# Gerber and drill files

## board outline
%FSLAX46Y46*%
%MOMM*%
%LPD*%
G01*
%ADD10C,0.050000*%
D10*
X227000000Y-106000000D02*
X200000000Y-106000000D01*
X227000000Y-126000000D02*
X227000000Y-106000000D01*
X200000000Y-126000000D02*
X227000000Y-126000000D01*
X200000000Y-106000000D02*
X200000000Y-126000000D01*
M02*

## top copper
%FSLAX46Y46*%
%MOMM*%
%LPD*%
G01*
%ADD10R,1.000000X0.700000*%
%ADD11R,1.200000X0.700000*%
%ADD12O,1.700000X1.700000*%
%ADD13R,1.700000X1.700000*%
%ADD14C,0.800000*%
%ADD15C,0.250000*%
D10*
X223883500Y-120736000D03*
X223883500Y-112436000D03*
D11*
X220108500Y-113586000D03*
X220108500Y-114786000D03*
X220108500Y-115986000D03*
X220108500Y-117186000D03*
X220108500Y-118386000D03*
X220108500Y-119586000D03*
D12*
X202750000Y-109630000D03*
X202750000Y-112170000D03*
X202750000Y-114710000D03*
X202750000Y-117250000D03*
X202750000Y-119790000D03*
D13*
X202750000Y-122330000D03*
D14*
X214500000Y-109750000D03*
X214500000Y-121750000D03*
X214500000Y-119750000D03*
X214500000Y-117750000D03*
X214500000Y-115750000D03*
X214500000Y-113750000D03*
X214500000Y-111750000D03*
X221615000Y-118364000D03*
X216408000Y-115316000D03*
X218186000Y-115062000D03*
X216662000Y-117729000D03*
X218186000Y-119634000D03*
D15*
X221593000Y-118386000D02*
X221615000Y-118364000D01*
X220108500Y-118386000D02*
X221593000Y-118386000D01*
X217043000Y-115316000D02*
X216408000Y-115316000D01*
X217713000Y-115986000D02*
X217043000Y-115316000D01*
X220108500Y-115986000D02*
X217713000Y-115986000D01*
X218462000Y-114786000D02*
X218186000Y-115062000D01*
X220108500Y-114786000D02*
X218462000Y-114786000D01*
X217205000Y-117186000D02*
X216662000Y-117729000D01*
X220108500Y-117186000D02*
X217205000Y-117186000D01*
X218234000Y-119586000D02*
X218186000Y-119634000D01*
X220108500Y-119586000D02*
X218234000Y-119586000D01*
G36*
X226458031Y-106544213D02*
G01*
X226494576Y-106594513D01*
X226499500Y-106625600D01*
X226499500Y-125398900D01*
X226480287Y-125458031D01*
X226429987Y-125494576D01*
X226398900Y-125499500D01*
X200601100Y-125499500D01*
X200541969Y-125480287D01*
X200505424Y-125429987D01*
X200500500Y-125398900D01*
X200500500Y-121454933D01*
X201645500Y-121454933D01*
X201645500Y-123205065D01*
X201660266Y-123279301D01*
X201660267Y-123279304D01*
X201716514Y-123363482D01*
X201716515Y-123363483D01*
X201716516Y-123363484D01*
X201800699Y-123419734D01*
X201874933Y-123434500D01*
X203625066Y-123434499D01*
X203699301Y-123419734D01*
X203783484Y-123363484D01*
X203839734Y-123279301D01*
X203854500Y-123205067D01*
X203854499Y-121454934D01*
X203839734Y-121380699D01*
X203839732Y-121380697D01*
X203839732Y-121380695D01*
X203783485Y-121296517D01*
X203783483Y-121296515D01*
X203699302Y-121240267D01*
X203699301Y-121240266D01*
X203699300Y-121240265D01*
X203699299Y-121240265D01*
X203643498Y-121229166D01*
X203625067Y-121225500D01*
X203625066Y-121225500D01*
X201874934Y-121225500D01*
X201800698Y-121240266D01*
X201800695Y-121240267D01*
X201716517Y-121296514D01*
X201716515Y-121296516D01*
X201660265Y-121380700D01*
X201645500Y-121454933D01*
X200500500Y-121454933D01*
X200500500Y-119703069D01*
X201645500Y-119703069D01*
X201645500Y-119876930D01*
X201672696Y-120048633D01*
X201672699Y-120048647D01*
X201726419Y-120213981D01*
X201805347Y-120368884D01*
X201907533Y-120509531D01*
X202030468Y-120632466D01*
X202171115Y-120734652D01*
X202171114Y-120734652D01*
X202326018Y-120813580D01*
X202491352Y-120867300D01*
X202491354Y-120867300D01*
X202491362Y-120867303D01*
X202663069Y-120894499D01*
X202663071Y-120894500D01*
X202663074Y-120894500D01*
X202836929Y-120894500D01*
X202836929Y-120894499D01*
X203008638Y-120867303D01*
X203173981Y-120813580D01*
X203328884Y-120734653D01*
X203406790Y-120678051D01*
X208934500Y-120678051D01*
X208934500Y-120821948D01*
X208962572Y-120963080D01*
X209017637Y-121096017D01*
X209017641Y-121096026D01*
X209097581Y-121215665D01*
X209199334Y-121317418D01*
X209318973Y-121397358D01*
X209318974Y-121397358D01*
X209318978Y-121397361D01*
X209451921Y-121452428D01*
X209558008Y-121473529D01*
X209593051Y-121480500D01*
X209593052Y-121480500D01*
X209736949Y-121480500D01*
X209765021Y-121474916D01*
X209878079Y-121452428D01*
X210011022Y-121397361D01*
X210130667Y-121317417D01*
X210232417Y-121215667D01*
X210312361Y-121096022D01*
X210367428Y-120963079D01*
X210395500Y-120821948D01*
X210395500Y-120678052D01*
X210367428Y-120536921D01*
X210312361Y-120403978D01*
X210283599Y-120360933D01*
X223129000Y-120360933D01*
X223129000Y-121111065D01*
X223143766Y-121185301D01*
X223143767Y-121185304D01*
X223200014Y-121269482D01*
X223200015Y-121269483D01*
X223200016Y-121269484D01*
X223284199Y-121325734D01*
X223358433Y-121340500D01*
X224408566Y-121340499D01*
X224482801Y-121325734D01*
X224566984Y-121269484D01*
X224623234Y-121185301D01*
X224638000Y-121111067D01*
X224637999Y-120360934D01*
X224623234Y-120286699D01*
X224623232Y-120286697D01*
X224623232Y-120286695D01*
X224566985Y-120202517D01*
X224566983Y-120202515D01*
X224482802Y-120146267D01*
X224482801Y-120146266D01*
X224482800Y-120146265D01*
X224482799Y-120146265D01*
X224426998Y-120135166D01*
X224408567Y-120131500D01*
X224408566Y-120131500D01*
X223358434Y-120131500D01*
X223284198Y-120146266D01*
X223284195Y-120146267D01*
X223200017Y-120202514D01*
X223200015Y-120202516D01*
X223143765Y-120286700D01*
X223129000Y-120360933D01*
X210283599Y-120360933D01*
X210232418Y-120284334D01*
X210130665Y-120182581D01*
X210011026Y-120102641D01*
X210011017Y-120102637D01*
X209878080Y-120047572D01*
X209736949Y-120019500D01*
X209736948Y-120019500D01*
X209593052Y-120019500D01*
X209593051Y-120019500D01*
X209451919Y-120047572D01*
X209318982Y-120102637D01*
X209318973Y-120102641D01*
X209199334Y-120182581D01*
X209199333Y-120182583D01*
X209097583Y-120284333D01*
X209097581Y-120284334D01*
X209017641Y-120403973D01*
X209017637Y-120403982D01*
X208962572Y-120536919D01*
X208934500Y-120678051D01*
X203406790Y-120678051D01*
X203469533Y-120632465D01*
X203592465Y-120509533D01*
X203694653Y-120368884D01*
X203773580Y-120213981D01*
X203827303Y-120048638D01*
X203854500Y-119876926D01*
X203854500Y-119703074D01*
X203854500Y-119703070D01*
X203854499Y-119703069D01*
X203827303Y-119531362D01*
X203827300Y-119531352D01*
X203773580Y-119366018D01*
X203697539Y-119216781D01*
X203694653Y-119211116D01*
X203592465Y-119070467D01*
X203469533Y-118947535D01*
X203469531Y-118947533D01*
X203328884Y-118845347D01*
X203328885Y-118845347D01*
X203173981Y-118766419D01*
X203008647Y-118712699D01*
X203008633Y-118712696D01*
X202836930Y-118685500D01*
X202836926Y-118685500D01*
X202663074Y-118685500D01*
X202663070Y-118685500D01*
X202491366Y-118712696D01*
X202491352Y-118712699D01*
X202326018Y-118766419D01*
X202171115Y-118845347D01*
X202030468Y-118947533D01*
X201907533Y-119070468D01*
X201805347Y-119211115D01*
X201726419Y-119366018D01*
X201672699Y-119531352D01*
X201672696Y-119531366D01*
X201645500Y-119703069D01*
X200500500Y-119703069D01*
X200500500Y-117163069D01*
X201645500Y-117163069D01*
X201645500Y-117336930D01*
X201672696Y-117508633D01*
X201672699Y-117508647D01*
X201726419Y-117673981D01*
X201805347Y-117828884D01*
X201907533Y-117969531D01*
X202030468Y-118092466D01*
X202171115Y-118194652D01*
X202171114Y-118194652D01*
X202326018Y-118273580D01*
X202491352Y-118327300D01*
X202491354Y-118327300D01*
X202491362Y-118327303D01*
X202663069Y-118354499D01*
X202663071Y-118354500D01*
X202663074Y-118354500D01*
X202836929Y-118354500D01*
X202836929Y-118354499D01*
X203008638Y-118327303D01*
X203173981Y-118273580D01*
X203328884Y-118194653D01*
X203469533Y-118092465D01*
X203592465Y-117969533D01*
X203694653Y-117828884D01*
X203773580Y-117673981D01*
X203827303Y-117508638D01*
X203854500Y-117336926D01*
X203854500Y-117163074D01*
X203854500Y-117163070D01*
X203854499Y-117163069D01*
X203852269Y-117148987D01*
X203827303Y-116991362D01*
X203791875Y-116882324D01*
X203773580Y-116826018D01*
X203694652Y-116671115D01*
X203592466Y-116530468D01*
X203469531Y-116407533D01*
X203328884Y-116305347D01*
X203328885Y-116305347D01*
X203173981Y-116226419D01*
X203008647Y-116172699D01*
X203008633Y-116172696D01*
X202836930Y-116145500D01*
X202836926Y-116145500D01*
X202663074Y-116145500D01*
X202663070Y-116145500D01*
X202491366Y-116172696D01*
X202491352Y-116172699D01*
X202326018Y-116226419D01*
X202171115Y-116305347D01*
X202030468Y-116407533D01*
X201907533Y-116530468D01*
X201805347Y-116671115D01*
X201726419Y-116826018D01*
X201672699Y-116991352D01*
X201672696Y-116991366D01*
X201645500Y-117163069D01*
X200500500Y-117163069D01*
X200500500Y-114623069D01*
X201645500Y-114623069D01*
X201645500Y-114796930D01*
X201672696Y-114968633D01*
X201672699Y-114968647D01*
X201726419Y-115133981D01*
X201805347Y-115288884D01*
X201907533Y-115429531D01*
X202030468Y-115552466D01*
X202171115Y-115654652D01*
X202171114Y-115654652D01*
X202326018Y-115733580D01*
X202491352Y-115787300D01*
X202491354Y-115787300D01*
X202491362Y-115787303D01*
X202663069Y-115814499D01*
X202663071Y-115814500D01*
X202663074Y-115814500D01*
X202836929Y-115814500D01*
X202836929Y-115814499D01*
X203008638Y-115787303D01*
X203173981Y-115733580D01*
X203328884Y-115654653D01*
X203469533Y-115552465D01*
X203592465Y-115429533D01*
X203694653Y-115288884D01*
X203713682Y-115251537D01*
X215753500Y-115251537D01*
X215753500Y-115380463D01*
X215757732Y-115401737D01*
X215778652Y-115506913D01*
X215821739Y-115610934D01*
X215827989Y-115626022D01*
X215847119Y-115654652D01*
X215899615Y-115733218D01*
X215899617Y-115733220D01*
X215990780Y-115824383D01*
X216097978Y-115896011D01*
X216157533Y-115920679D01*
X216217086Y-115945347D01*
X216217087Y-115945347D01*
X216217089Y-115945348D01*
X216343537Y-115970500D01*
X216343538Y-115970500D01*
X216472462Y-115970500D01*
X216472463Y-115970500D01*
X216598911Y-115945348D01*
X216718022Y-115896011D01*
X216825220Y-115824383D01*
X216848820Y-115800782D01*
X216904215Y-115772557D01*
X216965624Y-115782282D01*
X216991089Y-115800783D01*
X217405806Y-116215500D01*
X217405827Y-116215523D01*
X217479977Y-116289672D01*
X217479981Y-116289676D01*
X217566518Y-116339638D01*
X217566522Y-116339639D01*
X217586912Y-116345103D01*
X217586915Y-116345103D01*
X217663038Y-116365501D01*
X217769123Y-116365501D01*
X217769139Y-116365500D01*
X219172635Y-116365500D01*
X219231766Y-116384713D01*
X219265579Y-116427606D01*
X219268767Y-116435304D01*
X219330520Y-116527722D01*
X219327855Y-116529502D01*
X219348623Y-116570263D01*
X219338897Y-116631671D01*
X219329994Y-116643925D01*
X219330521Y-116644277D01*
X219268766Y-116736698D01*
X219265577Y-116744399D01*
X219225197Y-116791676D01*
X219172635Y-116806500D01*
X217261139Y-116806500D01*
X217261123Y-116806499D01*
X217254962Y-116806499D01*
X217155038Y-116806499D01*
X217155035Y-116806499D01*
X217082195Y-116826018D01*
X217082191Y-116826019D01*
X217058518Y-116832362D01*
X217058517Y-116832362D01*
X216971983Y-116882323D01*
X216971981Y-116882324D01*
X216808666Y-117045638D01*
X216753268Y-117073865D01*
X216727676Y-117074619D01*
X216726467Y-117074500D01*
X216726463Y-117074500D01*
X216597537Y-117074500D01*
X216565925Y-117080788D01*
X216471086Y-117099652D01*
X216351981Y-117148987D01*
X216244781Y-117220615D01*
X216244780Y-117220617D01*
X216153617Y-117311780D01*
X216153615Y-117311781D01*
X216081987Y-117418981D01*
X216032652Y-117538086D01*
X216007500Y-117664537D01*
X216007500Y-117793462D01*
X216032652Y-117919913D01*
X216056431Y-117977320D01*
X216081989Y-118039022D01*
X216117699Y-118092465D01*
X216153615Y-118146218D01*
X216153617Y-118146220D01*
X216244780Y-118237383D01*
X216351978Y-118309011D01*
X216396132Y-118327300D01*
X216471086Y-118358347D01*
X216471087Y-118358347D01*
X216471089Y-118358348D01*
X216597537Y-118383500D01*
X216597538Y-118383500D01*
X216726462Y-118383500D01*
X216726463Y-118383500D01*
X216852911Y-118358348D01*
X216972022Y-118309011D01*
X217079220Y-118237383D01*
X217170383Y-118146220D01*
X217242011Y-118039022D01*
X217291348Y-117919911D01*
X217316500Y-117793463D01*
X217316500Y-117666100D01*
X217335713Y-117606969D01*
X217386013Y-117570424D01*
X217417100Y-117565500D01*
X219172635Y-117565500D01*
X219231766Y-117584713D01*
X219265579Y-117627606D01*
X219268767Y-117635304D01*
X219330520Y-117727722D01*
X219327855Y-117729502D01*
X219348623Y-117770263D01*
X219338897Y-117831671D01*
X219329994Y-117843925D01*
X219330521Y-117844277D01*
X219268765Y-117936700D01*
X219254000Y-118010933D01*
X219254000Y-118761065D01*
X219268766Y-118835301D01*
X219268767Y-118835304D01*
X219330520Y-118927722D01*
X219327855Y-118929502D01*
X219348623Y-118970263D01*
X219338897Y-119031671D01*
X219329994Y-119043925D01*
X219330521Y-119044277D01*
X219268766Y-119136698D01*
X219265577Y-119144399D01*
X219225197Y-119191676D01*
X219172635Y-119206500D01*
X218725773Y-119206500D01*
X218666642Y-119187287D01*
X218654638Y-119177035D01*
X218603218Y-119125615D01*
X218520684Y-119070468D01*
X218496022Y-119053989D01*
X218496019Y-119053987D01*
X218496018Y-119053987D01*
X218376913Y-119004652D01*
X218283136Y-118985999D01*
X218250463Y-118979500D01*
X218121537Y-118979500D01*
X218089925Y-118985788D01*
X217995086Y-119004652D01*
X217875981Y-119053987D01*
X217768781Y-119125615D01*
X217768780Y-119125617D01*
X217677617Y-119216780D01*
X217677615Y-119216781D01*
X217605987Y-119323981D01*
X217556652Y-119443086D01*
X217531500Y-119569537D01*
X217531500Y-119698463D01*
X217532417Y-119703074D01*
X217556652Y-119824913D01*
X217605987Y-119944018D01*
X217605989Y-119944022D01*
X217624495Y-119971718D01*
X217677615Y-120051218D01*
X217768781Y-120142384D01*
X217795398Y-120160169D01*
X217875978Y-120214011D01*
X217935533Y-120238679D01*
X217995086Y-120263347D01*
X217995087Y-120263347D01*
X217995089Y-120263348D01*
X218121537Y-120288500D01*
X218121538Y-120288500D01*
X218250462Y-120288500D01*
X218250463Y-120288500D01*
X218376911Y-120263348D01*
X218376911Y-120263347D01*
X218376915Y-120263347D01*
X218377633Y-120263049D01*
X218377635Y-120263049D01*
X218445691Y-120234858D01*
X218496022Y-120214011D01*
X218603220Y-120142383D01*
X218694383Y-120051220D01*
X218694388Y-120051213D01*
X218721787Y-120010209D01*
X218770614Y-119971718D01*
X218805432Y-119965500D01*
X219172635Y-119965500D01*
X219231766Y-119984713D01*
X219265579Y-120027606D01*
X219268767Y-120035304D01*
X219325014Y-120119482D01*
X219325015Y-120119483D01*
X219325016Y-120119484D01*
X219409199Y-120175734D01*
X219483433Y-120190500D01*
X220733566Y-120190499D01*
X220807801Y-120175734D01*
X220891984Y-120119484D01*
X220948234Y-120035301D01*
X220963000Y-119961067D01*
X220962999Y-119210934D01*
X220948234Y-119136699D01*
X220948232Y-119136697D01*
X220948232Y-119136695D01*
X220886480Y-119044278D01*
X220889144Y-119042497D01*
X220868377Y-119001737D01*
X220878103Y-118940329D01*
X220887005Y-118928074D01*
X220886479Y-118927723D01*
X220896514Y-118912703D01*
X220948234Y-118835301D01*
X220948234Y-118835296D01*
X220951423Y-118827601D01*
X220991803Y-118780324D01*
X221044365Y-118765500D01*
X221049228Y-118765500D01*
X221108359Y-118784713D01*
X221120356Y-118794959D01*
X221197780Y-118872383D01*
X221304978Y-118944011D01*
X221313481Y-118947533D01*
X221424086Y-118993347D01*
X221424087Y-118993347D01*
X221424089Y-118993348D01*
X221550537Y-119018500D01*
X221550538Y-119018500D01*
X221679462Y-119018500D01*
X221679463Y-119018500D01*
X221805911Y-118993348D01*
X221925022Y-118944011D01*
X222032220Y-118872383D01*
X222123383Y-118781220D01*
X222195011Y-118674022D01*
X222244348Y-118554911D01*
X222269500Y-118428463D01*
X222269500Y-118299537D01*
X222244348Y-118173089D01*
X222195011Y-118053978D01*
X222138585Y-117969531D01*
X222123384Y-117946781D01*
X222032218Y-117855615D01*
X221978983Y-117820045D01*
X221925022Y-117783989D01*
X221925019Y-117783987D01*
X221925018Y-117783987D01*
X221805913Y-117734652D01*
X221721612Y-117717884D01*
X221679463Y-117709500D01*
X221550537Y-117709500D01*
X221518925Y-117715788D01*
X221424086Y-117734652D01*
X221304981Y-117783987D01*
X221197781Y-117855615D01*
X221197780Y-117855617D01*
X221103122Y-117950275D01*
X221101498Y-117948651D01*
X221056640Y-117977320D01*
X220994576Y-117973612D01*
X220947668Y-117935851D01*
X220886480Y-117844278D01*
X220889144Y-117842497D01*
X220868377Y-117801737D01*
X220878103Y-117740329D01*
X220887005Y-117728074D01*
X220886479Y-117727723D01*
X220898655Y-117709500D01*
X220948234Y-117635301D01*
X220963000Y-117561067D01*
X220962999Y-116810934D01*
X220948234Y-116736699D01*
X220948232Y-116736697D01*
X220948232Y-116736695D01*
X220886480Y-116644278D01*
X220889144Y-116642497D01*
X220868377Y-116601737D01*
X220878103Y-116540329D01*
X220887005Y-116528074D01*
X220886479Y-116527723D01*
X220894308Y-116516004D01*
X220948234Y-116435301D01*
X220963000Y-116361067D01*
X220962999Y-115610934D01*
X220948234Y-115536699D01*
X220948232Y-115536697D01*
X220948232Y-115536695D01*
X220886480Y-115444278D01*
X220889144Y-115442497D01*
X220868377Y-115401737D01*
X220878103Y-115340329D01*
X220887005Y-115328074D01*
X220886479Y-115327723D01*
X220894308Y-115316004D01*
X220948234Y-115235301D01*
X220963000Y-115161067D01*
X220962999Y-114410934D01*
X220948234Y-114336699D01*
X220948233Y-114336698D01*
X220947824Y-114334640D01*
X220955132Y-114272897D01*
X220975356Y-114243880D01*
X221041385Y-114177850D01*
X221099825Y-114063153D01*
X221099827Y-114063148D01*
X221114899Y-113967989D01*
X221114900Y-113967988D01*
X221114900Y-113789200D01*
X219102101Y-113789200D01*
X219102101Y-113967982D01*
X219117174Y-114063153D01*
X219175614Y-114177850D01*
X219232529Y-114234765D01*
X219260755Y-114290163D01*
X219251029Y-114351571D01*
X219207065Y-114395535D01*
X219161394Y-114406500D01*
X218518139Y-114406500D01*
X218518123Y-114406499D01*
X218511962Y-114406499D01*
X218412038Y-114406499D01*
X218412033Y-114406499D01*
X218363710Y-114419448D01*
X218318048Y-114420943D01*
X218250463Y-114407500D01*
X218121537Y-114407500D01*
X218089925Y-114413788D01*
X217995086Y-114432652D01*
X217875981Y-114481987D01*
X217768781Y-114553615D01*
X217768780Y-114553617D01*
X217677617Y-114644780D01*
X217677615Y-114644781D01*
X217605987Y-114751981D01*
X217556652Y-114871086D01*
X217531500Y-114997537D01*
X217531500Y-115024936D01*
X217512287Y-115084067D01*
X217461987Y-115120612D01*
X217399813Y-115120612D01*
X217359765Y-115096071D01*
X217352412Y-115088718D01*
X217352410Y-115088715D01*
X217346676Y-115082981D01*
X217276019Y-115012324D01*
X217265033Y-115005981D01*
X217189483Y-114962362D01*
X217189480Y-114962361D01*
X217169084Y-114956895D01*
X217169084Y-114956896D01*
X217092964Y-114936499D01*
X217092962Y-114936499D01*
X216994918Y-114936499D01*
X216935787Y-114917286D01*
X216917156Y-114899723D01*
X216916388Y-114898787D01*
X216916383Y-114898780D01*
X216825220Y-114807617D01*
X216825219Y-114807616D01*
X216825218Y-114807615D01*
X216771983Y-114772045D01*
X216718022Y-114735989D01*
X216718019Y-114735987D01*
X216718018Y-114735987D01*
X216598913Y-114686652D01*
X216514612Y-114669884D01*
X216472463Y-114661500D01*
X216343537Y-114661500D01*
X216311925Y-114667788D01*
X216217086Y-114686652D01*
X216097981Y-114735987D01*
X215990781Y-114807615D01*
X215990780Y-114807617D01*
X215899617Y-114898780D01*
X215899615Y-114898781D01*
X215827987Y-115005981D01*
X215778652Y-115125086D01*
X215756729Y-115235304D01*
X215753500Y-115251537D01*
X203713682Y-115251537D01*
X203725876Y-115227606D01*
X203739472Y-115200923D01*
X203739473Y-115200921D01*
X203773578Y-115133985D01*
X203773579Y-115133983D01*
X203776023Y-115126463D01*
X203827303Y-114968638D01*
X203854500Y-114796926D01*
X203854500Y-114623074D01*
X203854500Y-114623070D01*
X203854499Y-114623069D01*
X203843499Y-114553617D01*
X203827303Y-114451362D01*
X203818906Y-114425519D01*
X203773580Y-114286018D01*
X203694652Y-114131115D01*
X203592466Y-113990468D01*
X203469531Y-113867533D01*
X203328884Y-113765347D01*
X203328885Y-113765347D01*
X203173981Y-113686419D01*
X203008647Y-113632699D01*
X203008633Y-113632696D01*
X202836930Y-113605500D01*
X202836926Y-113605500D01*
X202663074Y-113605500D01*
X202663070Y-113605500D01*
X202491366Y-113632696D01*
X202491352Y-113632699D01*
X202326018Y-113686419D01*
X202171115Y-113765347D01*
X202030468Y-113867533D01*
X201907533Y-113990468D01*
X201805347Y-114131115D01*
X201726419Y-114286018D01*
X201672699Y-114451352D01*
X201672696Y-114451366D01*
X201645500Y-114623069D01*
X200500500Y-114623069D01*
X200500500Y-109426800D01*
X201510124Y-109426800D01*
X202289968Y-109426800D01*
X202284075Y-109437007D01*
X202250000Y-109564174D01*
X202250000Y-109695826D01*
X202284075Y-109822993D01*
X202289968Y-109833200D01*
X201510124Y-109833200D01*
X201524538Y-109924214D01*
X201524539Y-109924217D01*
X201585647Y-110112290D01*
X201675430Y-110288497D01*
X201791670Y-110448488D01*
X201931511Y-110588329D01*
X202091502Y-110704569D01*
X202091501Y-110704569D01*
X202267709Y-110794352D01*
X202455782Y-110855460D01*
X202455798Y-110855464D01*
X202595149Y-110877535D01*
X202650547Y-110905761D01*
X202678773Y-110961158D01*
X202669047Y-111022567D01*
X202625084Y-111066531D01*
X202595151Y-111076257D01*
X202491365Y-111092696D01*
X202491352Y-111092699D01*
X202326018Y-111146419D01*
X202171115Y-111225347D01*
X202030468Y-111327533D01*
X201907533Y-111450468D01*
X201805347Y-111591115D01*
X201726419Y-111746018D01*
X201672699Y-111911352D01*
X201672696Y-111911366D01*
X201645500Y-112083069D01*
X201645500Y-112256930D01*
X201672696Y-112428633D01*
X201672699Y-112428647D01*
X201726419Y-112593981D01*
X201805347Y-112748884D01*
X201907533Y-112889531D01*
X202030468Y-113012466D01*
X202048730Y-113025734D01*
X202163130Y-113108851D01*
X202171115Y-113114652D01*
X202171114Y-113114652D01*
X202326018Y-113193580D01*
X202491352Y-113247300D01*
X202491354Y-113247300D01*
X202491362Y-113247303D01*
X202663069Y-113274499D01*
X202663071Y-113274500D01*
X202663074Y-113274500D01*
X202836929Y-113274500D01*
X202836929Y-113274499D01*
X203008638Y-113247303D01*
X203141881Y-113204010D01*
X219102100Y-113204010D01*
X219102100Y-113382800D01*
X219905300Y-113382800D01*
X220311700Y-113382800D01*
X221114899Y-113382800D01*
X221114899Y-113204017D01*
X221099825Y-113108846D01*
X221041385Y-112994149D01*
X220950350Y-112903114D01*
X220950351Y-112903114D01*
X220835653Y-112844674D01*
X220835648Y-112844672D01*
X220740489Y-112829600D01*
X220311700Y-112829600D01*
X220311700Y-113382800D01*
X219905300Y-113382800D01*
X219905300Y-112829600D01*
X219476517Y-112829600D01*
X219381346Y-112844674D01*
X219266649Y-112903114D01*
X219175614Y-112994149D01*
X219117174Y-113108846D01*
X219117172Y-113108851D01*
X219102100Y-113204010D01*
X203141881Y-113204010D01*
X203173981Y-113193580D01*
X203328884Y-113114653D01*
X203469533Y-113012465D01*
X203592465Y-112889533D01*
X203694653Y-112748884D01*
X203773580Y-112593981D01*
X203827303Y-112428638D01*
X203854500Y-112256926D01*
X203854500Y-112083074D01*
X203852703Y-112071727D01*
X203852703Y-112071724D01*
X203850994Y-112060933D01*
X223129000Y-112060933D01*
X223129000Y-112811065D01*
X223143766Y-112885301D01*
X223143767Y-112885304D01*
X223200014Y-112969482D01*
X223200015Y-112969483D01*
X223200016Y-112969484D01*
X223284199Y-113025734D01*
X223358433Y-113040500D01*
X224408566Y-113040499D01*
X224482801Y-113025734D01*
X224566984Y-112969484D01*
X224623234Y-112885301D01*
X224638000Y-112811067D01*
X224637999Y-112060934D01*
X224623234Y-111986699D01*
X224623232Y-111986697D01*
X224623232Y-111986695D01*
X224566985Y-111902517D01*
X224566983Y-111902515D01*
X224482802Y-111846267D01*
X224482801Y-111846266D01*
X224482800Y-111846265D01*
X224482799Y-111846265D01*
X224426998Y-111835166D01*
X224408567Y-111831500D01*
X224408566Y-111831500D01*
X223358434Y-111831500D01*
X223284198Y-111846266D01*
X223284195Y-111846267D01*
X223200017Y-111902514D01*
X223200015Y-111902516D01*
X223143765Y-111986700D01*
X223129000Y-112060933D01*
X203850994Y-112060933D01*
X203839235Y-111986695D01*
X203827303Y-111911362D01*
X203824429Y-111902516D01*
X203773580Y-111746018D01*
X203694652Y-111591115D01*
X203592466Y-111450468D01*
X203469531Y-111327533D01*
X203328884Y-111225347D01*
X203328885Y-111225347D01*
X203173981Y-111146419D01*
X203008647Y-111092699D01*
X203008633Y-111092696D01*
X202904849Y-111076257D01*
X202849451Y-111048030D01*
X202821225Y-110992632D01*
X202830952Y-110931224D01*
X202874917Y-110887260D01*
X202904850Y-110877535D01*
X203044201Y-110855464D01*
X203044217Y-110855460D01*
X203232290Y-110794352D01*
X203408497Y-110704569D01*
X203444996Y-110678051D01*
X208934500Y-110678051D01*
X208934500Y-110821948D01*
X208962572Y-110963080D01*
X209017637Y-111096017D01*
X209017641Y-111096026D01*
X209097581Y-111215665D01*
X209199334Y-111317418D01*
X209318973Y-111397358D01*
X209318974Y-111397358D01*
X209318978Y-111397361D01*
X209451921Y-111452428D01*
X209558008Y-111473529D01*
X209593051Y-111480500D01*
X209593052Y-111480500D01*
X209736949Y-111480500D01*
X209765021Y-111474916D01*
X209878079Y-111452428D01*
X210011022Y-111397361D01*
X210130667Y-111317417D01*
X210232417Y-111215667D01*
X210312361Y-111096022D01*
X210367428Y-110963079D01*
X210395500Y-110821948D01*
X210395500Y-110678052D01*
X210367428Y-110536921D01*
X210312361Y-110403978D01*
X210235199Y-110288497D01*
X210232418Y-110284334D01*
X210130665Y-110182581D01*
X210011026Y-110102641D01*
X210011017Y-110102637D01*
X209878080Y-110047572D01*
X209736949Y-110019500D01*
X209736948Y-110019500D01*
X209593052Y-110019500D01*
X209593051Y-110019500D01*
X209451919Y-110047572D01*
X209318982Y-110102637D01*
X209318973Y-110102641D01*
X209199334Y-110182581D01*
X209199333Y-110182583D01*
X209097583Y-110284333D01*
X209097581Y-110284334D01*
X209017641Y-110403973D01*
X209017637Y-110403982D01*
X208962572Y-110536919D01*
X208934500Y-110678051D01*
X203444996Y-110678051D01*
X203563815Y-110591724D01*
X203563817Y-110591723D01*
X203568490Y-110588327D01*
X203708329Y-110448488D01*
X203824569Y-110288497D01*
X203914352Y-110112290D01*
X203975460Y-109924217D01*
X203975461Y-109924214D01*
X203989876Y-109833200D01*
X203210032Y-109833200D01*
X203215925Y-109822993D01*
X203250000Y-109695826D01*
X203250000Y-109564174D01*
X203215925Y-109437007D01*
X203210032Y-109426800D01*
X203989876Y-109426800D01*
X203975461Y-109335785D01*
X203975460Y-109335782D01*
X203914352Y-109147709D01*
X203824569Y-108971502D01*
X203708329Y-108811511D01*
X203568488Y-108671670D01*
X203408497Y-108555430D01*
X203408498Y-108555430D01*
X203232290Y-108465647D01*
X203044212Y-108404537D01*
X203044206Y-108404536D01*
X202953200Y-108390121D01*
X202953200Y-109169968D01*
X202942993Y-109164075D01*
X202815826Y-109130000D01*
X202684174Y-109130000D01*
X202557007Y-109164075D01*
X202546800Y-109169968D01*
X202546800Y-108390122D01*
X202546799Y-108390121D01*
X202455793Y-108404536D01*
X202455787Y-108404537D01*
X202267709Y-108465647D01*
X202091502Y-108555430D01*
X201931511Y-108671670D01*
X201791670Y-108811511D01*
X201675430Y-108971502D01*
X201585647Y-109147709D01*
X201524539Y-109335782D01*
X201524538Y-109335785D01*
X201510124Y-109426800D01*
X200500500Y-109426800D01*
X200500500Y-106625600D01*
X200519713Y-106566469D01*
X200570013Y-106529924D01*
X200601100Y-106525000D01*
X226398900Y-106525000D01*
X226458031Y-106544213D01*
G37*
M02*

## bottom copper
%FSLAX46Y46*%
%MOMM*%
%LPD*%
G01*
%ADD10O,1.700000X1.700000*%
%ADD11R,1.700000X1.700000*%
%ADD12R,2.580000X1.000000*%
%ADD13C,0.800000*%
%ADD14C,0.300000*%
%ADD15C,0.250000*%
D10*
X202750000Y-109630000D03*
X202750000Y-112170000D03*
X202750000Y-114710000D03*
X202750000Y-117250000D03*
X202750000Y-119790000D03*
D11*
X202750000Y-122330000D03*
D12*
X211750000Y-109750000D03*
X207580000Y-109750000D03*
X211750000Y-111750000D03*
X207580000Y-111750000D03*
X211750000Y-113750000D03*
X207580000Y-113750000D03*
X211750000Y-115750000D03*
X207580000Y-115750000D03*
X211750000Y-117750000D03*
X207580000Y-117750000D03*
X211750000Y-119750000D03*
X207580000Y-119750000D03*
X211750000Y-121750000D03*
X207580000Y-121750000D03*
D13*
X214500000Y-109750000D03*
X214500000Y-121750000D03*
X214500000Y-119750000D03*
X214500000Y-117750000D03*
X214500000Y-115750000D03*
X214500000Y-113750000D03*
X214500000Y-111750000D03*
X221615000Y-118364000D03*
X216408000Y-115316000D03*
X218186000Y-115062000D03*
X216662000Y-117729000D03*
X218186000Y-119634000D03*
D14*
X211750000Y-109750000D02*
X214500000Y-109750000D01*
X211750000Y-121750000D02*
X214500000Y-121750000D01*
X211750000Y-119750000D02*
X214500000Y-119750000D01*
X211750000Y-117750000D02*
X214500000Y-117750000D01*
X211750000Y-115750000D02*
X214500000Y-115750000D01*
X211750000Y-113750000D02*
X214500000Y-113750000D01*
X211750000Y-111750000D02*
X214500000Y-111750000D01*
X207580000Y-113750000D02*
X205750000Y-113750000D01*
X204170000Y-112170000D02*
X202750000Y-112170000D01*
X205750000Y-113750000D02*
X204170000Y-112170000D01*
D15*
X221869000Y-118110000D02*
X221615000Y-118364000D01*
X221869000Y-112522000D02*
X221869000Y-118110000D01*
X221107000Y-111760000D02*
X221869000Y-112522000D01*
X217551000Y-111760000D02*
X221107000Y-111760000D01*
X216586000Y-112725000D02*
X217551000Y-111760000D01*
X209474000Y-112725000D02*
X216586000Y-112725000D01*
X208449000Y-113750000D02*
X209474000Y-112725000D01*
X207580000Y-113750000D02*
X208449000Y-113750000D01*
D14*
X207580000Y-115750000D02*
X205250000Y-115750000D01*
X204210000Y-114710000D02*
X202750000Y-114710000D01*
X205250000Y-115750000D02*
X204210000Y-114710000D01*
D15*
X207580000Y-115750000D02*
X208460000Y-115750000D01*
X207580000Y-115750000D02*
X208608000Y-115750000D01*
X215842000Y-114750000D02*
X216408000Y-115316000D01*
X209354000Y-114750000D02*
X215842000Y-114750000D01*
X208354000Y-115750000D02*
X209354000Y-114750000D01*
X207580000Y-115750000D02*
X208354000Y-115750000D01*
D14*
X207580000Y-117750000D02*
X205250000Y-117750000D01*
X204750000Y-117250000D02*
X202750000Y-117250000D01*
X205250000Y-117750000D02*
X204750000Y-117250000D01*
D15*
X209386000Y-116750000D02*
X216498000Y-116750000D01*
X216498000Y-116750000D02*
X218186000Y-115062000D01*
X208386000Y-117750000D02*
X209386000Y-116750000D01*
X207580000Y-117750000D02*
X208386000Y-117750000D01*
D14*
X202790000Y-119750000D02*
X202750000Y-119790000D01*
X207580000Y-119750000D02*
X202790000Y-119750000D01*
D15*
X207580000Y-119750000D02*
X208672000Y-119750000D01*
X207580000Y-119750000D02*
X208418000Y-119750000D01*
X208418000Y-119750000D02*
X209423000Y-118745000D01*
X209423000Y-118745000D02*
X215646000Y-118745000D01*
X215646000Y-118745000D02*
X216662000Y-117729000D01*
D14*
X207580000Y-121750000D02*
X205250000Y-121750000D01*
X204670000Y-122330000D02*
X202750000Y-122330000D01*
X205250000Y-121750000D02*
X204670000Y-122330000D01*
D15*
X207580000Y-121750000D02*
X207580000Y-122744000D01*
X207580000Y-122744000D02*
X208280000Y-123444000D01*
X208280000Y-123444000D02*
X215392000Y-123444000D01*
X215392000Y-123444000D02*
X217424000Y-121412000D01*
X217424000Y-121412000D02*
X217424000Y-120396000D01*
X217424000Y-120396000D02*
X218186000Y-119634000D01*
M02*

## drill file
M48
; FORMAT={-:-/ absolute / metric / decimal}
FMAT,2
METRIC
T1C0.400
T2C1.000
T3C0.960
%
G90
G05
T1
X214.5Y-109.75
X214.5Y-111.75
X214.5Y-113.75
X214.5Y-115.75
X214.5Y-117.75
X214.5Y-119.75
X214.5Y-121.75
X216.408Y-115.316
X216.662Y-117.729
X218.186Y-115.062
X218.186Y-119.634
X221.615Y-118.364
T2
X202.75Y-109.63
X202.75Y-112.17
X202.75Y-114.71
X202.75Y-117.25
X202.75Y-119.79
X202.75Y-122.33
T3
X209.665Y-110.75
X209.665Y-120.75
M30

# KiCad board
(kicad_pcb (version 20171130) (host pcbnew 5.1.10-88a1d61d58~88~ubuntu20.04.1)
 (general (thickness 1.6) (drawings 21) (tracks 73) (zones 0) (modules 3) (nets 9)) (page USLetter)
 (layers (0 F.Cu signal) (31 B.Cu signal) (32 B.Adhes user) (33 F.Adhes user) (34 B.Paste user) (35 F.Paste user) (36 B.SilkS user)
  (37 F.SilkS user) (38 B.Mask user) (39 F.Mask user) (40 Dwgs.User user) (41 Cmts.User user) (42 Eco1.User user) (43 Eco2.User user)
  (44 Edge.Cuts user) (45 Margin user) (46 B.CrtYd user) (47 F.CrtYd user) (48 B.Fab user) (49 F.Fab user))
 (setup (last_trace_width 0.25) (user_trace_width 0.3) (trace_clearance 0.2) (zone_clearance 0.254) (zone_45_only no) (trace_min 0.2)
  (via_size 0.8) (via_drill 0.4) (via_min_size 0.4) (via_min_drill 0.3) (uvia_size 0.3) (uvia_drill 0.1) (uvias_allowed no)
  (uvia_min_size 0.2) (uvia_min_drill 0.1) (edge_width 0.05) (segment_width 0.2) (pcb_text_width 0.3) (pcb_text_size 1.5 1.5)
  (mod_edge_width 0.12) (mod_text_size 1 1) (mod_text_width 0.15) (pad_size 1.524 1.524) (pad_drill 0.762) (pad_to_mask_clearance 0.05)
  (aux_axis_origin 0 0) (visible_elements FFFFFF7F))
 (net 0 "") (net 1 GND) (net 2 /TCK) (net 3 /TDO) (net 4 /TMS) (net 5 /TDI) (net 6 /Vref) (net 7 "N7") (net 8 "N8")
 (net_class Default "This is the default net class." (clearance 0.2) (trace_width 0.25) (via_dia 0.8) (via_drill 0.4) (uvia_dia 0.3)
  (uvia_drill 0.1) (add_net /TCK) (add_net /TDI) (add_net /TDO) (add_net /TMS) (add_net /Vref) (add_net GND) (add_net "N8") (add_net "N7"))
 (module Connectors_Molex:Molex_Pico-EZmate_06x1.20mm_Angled (layer F.Cu) (at 221.996 116.586 90)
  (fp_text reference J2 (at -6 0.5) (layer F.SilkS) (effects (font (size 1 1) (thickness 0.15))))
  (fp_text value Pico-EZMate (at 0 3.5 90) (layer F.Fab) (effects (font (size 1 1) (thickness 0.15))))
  (pad "" smd rect (at -4.15 1.8875 90) (size 0.7 1) (layers F.Cu F.Paste F.Mask))
  (pad "" smd rect (at 4.15 1.8875 90) (size 0.7 1) (layers F.Cu F.Paste F.Mask))
  (pad 6 smd rect (at 3 -1.8875 90) (size 0.7 1.2) (layers F.Cu F.Paste F.Mask) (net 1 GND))
  (pad 5 smd rect (at 1.8 -1.8875 90) (size 0.7 1.2) (layers F.Cu F.Paste F.Mask) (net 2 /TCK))
  (pad 4 smd rect (at 0.6 -1.8875 90) (size 0.7 1.2) (layers F.Cu F.Paste F.Mask) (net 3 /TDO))
  (pad 3 smd rect (at -0.6 -1.8875 90) (size 0.7 1.2) (layers F.Cu F.Paste F.Mask) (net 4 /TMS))
  (pad 2 smd rect (at -1.8 -1.8875 90) (size 0.7 1.2) (layers F.Cu F.Paste F.Mask) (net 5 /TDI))
  (pad 1 smd rect (at -3 -1.8875 90) (size 0.7 1.2) (layers F.Cu F.Paste F.Mask) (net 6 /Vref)))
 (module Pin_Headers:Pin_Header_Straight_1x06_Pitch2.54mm (layer B.Cu) (at 202.75 122.33)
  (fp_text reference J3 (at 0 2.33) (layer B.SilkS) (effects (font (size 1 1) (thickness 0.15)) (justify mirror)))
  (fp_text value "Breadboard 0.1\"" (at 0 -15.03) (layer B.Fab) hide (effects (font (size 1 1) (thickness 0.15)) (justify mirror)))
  (pad 6 thru_hole oval (at 0 -12.7) (size 1.7 1.7) (drill 1) (layers *.Cu *.Mask) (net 1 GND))
  (pad 5 thru_hole oval (at 0 -10.16) (size 1.7 1.7) (drill 1) (layers *.Cu *.Mask) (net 5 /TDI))
  (pad 4 thru_hole oval (at 0 -7.62) (size 1.7 1.7) (drill 1) (layers *.Cu *.Mask) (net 3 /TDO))
  (pad 3 thru_hole oval (at 0 -5.08) (size 1.7 1.7) (drill 1) (layers *.Cu *.Mask) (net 2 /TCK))
  (pad 2 thru_hole oval (at 0 -2.54) (size 1.7 1.7) (drill 1) (layers *.Cu *.Mask) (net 4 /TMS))
  (pad 1 thru_hole rect (at 0 0) (size 1.7 1.7) (drill 1) (layers *.Cu *.Mask) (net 6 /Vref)))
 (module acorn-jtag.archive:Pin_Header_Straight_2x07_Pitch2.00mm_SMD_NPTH (layer B.Cu) (at 209.665 115.75)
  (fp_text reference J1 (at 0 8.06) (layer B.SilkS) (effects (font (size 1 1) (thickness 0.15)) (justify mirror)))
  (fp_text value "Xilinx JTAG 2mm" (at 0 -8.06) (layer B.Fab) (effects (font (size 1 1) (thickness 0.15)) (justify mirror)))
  (pad 14 smd rect (at 2.085 -6) (size 2.58 1) (layers B.Cu B.Paste B.Mask) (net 1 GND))
  (pad 13 smd rect (at -2.085 -6) (size 2.58 1) (layers B.Cu B.Paste B.Mask) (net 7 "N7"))
  (pad 12 smd rect (at 2.085 -4) (size 2.58 1) (layers B.Cu B.Paste B.Mask) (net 1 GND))
  (pad 11 smd rect (at -2.085 -4) (size 2.58 1) (layers B.Cu B.Paste B.Mask) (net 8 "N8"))
  (pad 10 smd rect (at 2.085 -2) (size 2.58 1) (layers B.Cu B.Paste B.Mask) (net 1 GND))
  (pad 9 smd rect (at -2.085 -2) (size 2.58 1) (layers B.Cu B.Paste B.Mask) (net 5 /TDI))
  (pad 8 smd rect (at 2.085 0) (size 2.58 1) (layers B.Cu B.Paste B.Mask) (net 1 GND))
  (pad 7 smd rect (at -2.085 0) (size 2.58 1) (layers B.Cu B.Paste B.Mask) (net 3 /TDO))
  (pad 6 smd rect (at 2.085 2) (size 2.58 1) (layers B.Cu B.Paste B.Mask) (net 1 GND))
  (pad 5 smd rect (at -2.085 2) (size 2.58 1) (layers B.Cu B.Paste B.Mask) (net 2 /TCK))
  (pad 4 smd rect (at 2.085 4) (size 2.58 1) (layers B.Cu B.Paste B.Mask) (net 1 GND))
  (pad 3 smd rect (at -2.085 4) (size 2.58 1) (layers B.Cu B.Paste B.Mask) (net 4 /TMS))
  (pad 2 smd rect (at 2.085 6) (size 2.58 1) (layers B.Cu B.Paste B.Mask) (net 1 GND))
  (pad 1 smd rect (at -2.085 6) (size 2.58 1) (layers B.Cu B.Paste B.Mask) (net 6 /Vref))
  (pad "" np_thru_hole circle (at 0 5) (size 0.96 0.96) (drill 0.96) (layers *.Cu *.Mask))
  (pad "" np_thru_hole circle (at 0 -5) (size 0.96 0.96) (drill 0.96) (layers *.Cu *.Mask)))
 (gr_line (start 227 106) (end 200 106) (layer Edge.Cuts) (width 0.05))
 (gr_line (start 227 126) (end 227 106) (layer Edge.Cuts) (width 0.05))
 (gr_line (start 200 126) (end 227 126) (layer Edge.Cuts) (width 0.05))
 (gr_line (start 200 106) (end 200 126) (layer Edge.Cuts) (width 0.05))
 (segment (start 211.75 109.75) (end 214.5 109.75) (width 0.3) (layer B.Cu) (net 1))
 (via (at 214.5 109.75) (size 0.8) (drill 0.4) (layers F.Cu B.Cu) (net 1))
 (segment (start 211.75 121.75) (end 214.5 121.75) (width 0.3) (layer B.Cu) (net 1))
 (via (at 214.5 121.75) (size 0.8) (drill 0.4) (layers F.Cu B.Cu) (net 1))
 (segment (start 211.75 119.75) (end 214.5 119.75) (width 0.3) (layer B.Cu) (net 1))
 (via (at 214.5 119.75) (size 0.8) (drill 0.4) (layers F.Cu B.Cu) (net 1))
 (segment (start 211.75 117.75) (end 214.5 117.75) (width 0.3) (layer B.Cu) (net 1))
 (via (at 214.5 117.75) (size 0.8) (drill 0.4) (layers F.Cu B.Cu) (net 1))
 (segment (start 211.75 115.75) (end 214.5 115.75) (width 0.3) (layer B.Cu) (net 1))
 (via (at 214.5 115.75) (size 0.8) (drill 0.4) (layers F.Cu B.Cu) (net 1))
 (segment (start 211.75 113.75) (end 214.5 113.75) (width 0.3) (layer B.Cu) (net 1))
 (via (at 214.5 113.75) (size 0.8) (drill 0.4) (layers F.Cu B.Cu) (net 1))
 (segment (start 211.75 111.75) (end 214.5 111.75) (width 0.3) (layer B.Cu) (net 1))
 (via (at 214.5 111.75) (size 0.8) (drill 0.4) (layers F.Cu B.Cu) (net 1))
 (segment (start 207.58 113.75) (end 205.75 113.75) (width 0.3) (layer B.Cu) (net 5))
 (segment (start 204.17 112.17) (end 202.75 112.17) (width 0.3) (layer B.Cu) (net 5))
 (segment (start 205.75 113.75) (end 204.17 112.17) (width 0.3) (layer B.Cu) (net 5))
 (via (at 221.615 118.364) (size 0.8) (drill 0.4) (layers F.Cu B.Cu) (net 5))
 (segment (start 221.593 118.386) (end 221.615 118.364) (width 0.25) (layer F.Cu) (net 5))
 (segment (start 220.1085 118.386) (end 221.593 118.386) (width 0.25) (layer F.Cu) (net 5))
 (segment (start 221.869 118.11) (end 221.615 118.364) (width 0.25) (layer B.Cu) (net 5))
 (segment (start 221.869 112.522) (end 221.869 118.11) (width 0.25) (layer B.Cu) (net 5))
 (segment (start 221.107 111.76) (end 221.869 112.522) (width 0.25) (layer B.Cu) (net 5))
 (segment (start 217.551 111.76) (end 221.107 111.76) (width 0.25) (layer B.Cu) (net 5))
 (segment (start 216.586 112.725) (end 217.551 111.76) (width 0.25) (layer B.Cu) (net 5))
 (segment (start 209.474 112.725) (end 216.586 112.725) (width 0.25) (layer B.Cu) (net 5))
 (segment (start 208.449 113.75) (end 209.474 112.725) (width 0.25) (layer B.Cu) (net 5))
 (segment (start 207.58 113.75) (end 208.449 113.75) (width 0.25) (layer B.Cu) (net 5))
 (segment (start 207.58 115.75) (end 205.25 115.75) (width 0.3) (layer B.Cu) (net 3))
 (segment (start 204.21 114.71) (end 202.75 114.71) (width 0.3) (layer B.Cu) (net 3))
 (segment (start 205.25 115.75) (end 204.21 114.71) (width 0.3) (layer B.Cu) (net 3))
 (segment (start 207.58 115.75) (end 208.46 115.75) (width 0.25) (layer B.Cu) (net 3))
 (segment (start 207.58 115.75) (end 208.608 115.75) (width 0.25) (layer B.Cu) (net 3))
 (via (at 216.408 115.316) (size 0.8) (drill 0.4) (layers F.Cu B.Cu) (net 3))
 (segment (start 217.043 115.316) (end 216.408 115.316) (width 0.25) (layer F.Cu) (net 3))
 (segment (start 217.713 115.986) (end 217.043 115.316) (width 0.25) (layer F.Cu) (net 3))
 (segment (start 220.1085 115.986) (end 217.713 115.986) (width 0.25) (layer F.Cu) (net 3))
 (segment (start 215.842 114.75) (end 216.408 115.316) (width 0.25) (layer B.Cu) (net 3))
 (segment (start 209.354 114.75) (end 215.842 114.75) (width 0.25) (layer B.Cu) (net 3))
 (segment (start 208.354 115.75) (end 209.354 114.75) (width 0.25) (layer B.Cu) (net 3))
 (segment (start 207.58 115.75) (end 208.354 115.75) (width 0.25) (layer B.Cu) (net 3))
 (segment (start 207.58 117.75) (end 205.25 117.75) (width 0.3) (layer B.Cu) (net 2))
 (segment (start 204.75 117.25) (end 202.75 117.25) (width 0.3) (layer B.Cu) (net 2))
 (segment (start 205.25 117.75) (end 204.75 117.25) (width 0.3) (layer B.Cu) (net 2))
 (via (at 218.186 115.062) (size 0.8) (drill 0.4) (layers F.Cu B.Cu) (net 2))
 (segment (start 218.462 114.786) (end 218.186 115.062) (width 0.25) (layer F.Cu) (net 2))
 (segment (start 220.1085 114.786) (end 218.462 114.786) (width 0.25) (layer F.Cu) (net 2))
 (segment (start 209.386 116.75) (end 216.498 116.75) (width 0.25) (layer B.Cu) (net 2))
 (segment (start 216.498 116.75) (end 218.186 115.062) (width 0.25) (layer B.Cu) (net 2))
 (segment (start 208.386 117.75) (end 209.386 116.75) (width 0.25) (layer B.Cu) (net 2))
 (segment (start 207.58 117.75) (end 208.386 117.75) (width 0.25) (layer B.Cu) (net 2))
 (segment (start 202.79 119.75) (end 202.75 119.79) (width 0.3) (layer B.Cu) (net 4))
 (segment (start 207.58 119.75) (end 202.79 119.75) (width 0.3) (layer B.Cu) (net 4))
 (segment (start 207.58 119.75) (end 208.672 119.75) (width 0.25) (layer B.Cu) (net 4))
 (segment (start 207.58 119.75) (end 208.418 119.75) (width 0.25) (layer B.Cu) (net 4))
 (segment (start 208.418 119.75) (end 209.423 118.745) (width 0.25) (layer B.Cu) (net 4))
 (segment (start 209.423 118.745) (end 215.646 118.745) (width 0.25) (layer B.Cu) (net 4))
 (segment (start 215.646 118.745) (end 216.662 117.729) (width 0.25) (layer B.Cu) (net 4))
 (via (at 216.662 117.729) (size 0.8) (drill 0.4) (layers F.Cu B.Cu) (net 4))
 (segment (start 217.205 117.186) (end 216.662 117.729) (width 0.25) (layer F.Cu) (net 4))
 (segment (start 220.1085 117.186) (end 217.205 117.186) (width 0.25) (layer F.Cu) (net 4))
 (segment (start 207.58 121.75) (end 205.25 121.75) (width 0.3) (layer B.Cu) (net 6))
 (segment (start 204.67 122.33) (end 202.75 122.33) (width 0.3) (layer B.Cu) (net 6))
 (segment (start 205.25 121.75) (end 204.67 122.33) (width 0.3) (layer B.Cu) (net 6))
 (segment (start 207.58 121.75) (end 207.58 122.744) (width 0.25) (layer B.Cu) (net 6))
 (segment (start 207.58 122.744) (end 208.28 123.444) (width 0.25) (layer B.Cu) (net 6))
 (segment (start 208.28 123.444) (end 215.392 123.444) (width 0.25) (layer B.Cu) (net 6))
 (segment (start 215.392 123.444) (end 217.424 121.412) (width 0.25) (layer B.Cu) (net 6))
 (segment (start 217.424 121.412) (end 217.424 120.396) (width 0.25) (layer B.Cu) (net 6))
 (segment (start 217.424 120.396) (end 218.186 119.634) (width 0.25) (layer B.Cu) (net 6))
 (via (at 218.186 119.634) (size 0.8) (drill 0.4) (layers F.Cu B.Cu) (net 6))
 (segment (start 218.234 119.586) (end 218.186 119.634) (width 0.25) (layer F.Cu) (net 6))
 (segment (start 220.1085 119.586) (end 218.234 119.586) (width 0.25) (layer F.Cu) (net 6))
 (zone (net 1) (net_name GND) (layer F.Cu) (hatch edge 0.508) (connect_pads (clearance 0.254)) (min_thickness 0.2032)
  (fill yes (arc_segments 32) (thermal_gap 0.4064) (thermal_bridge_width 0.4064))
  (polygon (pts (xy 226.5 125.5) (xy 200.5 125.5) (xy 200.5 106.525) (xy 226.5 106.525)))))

